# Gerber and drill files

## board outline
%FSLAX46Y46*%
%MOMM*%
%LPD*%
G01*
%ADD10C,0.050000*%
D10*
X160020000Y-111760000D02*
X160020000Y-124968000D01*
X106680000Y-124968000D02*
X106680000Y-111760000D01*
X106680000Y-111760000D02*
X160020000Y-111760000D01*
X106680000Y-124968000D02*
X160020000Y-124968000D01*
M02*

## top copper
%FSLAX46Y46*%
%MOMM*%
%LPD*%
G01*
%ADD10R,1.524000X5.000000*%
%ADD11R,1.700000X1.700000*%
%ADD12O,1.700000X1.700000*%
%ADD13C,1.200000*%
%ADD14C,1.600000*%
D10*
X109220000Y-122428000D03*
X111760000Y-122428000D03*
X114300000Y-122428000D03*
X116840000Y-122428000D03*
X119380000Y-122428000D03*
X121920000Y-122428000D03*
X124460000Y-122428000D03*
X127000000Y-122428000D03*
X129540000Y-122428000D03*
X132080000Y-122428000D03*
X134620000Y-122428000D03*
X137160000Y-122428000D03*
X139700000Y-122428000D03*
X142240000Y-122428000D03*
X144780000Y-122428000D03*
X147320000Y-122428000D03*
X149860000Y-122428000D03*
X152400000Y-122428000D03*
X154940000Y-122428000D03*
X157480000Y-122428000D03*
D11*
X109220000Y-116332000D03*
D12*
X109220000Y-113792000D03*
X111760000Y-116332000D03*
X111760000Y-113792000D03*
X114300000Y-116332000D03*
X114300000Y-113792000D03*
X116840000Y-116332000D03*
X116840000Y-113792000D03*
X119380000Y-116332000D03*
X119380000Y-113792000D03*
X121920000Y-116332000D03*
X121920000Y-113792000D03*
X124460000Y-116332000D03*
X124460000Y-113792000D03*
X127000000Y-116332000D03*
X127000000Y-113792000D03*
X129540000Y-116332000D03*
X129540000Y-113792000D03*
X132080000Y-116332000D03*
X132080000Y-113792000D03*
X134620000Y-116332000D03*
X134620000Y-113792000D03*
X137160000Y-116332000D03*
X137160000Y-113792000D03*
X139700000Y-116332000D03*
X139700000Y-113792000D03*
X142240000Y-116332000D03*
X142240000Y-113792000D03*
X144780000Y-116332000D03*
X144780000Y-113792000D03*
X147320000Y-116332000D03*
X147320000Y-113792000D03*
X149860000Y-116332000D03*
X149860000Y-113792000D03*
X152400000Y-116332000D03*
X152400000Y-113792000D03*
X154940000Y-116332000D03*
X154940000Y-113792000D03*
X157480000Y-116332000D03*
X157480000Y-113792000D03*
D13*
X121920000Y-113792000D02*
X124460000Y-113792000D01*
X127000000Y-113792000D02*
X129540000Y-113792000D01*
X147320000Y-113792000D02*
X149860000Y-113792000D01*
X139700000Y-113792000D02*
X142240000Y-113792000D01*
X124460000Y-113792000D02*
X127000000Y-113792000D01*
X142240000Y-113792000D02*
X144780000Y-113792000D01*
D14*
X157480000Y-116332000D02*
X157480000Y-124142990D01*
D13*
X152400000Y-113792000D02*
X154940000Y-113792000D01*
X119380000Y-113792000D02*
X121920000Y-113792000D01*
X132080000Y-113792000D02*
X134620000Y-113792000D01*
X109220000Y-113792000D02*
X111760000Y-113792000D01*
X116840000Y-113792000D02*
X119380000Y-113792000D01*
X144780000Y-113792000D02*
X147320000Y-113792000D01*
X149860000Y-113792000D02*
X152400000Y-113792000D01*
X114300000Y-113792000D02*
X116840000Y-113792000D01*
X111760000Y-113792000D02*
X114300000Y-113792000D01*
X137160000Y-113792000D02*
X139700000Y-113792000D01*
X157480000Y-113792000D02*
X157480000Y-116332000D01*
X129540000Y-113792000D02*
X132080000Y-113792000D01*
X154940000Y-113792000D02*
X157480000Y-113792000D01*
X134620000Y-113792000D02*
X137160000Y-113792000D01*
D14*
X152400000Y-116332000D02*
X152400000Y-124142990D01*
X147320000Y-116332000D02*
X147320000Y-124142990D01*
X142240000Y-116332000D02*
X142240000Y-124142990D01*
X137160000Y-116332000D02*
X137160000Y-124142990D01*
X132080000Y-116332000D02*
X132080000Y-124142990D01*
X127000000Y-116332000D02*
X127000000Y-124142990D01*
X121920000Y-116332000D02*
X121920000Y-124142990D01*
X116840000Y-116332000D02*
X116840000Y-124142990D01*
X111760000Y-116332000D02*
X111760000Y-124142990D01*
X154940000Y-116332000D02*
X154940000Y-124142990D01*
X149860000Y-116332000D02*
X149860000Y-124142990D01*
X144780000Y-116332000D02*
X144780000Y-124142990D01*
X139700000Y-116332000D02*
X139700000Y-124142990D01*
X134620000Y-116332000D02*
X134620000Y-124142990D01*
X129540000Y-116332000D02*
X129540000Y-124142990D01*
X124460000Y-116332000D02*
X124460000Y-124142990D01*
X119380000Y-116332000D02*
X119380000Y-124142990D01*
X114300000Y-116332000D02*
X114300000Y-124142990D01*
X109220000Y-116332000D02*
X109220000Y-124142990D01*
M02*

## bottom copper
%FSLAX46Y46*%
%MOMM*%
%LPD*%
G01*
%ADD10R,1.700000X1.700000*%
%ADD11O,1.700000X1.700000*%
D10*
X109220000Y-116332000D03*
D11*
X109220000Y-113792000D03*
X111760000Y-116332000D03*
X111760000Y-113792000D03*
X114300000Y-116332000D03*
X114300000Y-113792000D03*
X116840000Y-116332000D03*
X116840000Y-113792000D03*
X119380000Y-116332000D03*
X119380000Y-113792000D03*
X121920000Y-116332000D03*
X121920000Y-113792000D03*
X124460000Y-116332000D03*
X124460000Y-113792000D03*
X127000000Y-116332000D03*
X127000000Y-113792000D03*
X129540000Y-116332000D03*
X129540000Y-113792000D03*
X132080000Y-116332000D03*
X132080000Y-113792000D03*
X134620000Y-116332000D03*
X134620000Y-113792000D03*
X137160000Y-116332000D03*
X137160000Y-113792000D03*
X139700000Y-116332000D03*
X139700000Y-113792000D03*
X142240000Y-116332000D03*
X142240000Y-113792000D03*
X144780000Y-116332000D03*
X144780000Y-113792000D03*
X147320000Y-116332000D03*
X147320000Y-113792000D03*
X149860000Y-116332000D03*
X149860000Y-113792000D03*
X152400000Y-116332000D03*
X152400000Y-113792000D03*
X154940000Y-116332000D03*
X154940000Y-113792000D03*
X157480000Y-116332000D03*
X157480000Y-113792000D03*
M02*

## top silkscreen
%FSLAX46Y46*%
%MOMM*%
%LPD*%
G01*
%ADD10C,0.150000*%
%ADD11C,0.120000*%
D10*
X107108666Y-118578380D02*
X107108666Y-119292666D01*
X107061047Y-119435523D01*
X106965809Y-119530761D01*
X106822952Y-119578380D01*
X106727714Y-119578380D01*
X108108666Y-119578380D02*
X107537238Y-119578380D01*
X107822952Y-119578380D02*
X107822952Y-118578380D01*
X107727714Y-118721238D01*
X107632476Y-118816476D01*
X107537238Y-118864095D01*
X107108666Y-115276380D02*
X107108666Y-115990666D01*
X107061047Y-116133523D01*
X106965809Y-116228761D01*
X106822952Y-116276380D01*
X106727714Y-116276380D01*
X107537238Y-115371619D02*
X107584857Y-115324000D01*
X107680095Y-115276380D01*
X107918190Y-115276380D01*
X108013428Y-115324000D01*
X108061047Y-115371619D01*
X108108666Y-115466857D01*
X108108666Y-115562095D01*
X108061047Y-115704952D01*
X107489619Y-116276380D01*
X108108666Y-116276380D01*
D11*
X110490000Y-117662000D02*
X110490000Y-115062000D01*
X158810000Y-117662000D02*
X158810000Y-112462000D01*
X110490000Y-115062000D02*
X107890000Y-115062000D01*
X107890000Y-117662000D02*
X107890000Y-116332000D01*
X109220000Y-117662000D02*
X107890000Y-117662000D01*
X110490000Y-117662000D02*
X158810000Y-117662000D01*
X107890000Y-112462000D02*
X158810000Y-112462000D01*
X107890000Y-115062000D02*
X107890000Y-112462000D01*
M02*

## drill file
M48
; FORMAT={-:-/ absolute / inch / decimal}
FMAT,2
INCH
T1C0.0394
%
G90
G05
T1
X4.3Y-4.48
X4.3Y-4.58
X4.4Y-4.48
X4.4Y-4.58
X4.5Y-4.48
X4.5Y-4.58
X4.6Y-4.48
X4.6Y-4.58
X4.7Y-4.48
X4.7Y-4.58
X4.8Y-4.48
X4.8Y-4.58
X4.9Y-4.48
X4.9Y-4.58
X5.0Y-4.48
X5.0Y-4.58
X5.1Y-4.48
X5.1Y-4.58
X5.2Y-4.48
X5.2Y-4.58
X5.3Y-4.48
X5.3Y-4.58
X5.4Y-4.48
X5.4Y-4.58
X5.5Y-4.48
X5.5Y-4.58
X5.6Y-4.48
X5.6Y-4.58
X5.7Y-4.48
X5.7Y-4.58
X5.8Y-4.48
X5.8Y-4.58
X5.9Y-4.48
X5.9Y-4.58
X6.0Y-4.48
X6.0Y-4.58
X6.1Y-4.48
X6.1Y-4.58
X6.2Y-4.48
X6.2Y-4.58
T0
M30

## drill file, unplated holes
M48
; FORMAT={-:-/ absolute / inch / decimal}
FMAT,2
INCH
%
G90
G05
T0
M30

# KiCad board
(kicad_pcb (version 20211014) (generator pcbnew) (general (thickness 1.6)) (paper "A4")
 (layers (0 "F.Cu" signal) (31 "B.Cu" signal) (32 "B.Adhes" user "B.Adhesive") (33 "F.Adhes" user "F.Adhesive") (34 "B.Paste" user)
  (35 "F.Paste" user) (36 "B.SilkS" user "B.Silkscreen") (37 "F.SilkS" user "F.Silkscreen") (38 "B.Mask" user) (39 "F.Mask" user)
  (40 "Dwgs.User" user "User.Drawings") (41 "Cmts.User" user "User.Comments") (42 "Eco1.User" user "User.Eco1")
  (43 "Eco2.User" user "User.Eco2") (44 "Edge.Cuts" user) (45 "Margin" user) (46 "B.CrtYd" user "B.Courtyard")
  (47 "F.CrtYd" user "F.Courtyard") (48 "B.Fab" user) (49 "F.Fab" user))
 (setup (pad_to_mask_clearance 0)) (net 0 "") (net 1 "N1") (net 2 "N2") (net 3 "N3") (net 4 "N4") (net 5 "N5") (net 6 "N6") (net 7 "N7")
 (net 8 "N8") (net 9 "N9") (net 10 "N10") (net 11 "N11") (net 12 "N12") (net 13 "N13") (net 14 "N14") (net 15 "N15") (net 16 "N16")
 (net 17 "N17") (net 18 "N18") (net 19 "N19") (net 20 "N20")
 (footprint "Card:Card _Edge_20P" (layer "F.Cu") (at 116.84 124.968)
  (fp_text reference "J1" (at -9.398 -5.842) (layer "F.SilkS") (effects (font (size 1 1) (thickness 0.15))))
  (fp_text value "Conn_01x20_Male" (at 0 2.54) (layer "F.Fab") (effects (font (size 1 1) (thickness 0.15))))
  (pad "1" smd rect locked (at -7.62 -2.54) (size 1.524 5) (layers "F.Cu" "F.Paste" "F.Mask") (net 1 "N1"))
  (pad "2" smd rect locked (at -5.08 -2.54) (size 1.524 5) (layers "F.Cu" "F.Paste" "F.Mask") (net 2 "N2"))
  (pad "3" smd rect locked (at -2.54 -2.54) (size 1.524 5) (layers "F.Cu" "F.Paste" "F.Mask") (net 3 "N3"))
  (pad "4" smd rect locked (at 0 -2.54) (size 1.524 5) (layers "F.Cu" "F.Paste" "F.Mask") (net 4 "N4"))
  (pad "5" smd rect locked (at 2.54 -2.54) (size 1.524 5) (layers "F.Cu" "F.Paste" "F.Mask") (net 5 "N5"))
  (pad "6" smd rect locked (at 5.08 -2.54) (size 1.524 5) (layers "F.Cu" "F.Paste" "F.Mask") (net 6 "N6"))
  (pad "7" smd rect locked (at 7.62 -2.54) (size 1.524 5) (layers "F.Cu" "F.Paste" "F.Mask") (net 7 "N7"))
  (pad "8" smd rect locked (at 10.16 -2.54) (size 1.524 5) (layers "F.Cu" "F.Paste" "F.Mask") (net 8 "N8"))
  (pad "9" smd rect locked (at 12.7 -2.54) (size 1.524 5) (layers "F.Cu" "F.Paste" "F.Mask") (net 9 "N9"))
  (pad "10" smd rect locked (at 15.24 -2.54) (size 1.524 5) (layers "F.Cu" "F.Paste" "F.Mask") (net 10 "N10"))
  (pad "11" smd rect locked (at 17.78 -2.54) (size 1.524 5) (layers "F.Cu" "F.Paste" "F.Mask") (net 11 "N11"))
  (pad "12" smd rect locked (at 20.32 -2.54) (size 1.524 5) (layers "F.Cu" "F.Paste" "F.Mask") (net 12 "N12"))
  (pad "13" smd rect locked (at 22.86 -2.54) (size 1.524 5) (layers "F.Cu" "F.Paste" "F.Mask") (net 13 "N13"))
  (pad "14" smd rect locked (at 25.4 -2.54) (size 1.524 5) (layers "F.Cu" "F.Paste" "F.Mask") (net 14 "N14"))
  (pad "15" smd rect locked (at 27.94 -2.54) (size 1.524 5) (layers "F.Cu" "F.Paste" "F.Mask") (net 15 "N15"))
  (pad "16" smd rect locked (at 30.48 -2.54) (size 1.524 5) (layers "F.Cu" "F.Paste" "F.Mask") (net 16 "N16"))
  (pad "17" smd rect locked (at 33.02 -2.54) (size 1.524 5) (layers "F.Cu" "F.Paste" "F.Mask") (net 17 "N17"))
  (pad "18" smd rect locked (at 35.56 -2.54) (size 1.524 5) (layers "F.Cu" "F.Paste" "F.Mask") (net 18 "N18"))
  (pad "19" smd rect locked (at 38.1 -2.54) (size 1.524 5) (layers "F.Cu" "F.Paste" "F.Mask") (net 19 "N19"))
  (pad "20" smd rect locked (at 40.64 -2.54) (size 1.524 5) (layers "F.Cu" "F.Paste" "F.Mask") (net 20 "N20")))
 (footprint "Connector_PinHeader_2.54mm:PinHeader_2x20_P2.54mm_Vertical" (layer "F.Cu") (at 109.22 116.332 90)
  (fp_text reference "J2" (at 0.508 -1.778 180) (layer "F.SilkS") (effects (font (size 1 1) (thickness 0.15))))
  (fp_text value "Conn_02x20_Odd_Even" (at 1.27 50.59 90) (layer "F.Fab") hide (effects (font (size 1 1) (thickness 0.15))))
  (fp_line (start -1.33 1.27) (end 1.27 1.27) (layer "F.SilkS") (width 0.12))
  (fp_line (start -1.33 49.59) (end 3.87 49.59) (layer "F.SilkS") (width 0.12))
  (fp_line (start 1.27 1.27) (end 1.27 -1.33) (layer "F.SilkS") (width 0.12))
  (fp_line (start -1.33 -1.33) (end 0 -1.33) (layer "F.SilkS") (width 0.12))
  (fp_line (start -1.33 0) (end -1.33 -1.33) (layer "F.SilkS") (width 0.12))
  (fp_line (start -1.33 1.27) (end -1.33 49.59) (layer "F.SilkS") (width 0.12))
  (fp_line (start 3.87 -1.33) (end 3.87 49.59) (layer "F.SilkS") (width 0.12))
  (fp_line (start 1.27 -1.33) (end 3.87 -1.33) (layer "F.SilkS") (width 0.12))
  (pad "1" thru_hole rect locked (at 0 0 90) (size 1.7 1.7) (drill 1) (layers *.Cu *.Mask) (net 1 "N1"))
  (pad "2" thru_hole oval locked (at 2.54 0 90) (size 1.7 1.7) (drill 1) (layers *.Cu *.Mask) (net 20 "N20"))
  (pad "3" thru_hole oval locked (at 0 2.54 90) (size 1.7 1.7) (drill 1) (layers *.Cu *.Mask) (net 2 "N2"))
  (pad "4" thru_hole oval locked (at 2.54 2.54 90) (size 1.7 1.7) (drill 1) (layers *.Cu *.Mask) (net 20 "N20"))
  (pad "5" thru_hole oval locked (at 0 5.08 90) (size 1.7 1.7) (drill 1) (layers *.Cu *.Mask) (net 3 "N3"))
  (pad "6" thru_hole oval locked (at 2.54 5.08 90) (size 1.7 1.7) (drill 1) (layers *.Cu *.Mask) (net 20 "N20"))
  (pad "7" thru_hole oval locked (at 0 7.62 90) (size 1.7 1.7) (drill 1) (layers *.Cu *.Mask) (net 4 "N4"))
  (pad "8" thru_hole oval locked (at 2.54 7.62 90) (size 1.7 1.7) (drill 1) (layers *.Cu *.Mask) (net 20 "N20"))
  (pad "9" thru_hole oval locked (at 0 10.16 90) (size 1.7 1.7) (drill 1) (layers *.Cu *.Mask) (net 5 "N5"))
  (pad "10" thru_hole oval locked (at 2.54 10.16 90) (size 1.7 1.7) (drill 1) (layers *.Cu *.Mask) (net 20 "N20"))
  (pad "11" thru_hole oval locked (at 0 12.7 90) (size 1.7 1.7) (drill 1) (layers *.Cu *.Mask) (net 6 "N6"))
  (pad "12" thru_hole oval locked (at 2.54 12.7 90) (size 1.7 1.7) (drill 1) (layers *.Cu *.Mask) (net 20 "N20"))
  (pad "13" thru_hole oval locked (at 0 15.24 90) (size 1.7 1.7) (drill 1) (layers *.Cu *.Mask) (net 7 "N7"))
  (pad "14" thru_hole oval locked (at 2.54 15.24 90) (size 1.7 1.7) (drill 1) (layers *.Cu *.Mask) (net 20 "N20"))
  (pad "15" thru_hole oval locked (at 0 17.78 90) (size 1.7 1.7) (drill 1) (layers *.Cu *.Mask) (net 8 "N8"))
  (pad "16" thru_hole oval locked (at 2.54 17.78 90) (size 1.7 1.7) (drill 1) (layers *.Cu *.Mask) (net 20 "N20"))
  (pad "17" thru_hole oval locked (at 0 20.32 90) (size 1.7 1.7) (drill 1) (layers *.Cu *.Mask) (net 9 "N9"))
  (pad "18" thru_hole oval locked (at 2.54 20.32 90) (size 1.7 1.7) (drill 1) (layers *.Cu *.Mask) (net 20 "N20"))
  (pad "19" thru_hole oval locked (at 0 22.86 90) (size 1.7 1.7) (drill 1) (layers *.Cu *.Mask) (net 10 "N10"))
  (pad "20" thru_hole oval locked (at 2.54 22.86 90) (size 1.7 1.7) (drill 1) (layers *.Cu *.Mask) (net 20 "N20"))
  (pad "21" thru_hole oval locked (at 0 25.4 90) (size 1.7 1.7) (drill 1) (layers *.Cu *.Mask) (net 11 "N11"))
  (pad "22" thru_hole oval locked (at 2.54 25.4 90) (size 1.7 1.7) (drill 1) (layers *.Cu *.Mask) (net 20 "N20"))
  (pad "23" thru_hole oval locked (at 0 27.94 90) (size 1.7 1.7) (drill 1) (layers *.Cu *.Mask) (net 12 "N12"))
  (pad "24" thru_hole oval locked (at 2.54 27.94 90) (size 1.7 1.7) (drill 1) (layers *.Cu *.Mask) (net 20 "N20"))
  (pad "25" thru_hole oval locked (at 0 30.48 90) (size 1.7 1.7) (drill 1) (layers *.Cu *.Mask) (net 13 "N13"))
  (pad "26" thru_hole oval locked (at 2.54 30.48 90) (size 1.7 1.7) (drill 1) (layers *.Cu *.Mask) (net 20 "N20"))
  (pad "27" thru_hole oval locked (at 0 33.02 90) (size 1.7 1.7) (drill 1) (layers *.Cu *.Mask) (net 14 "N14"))
  (pad "28" thru_hole oval locked (at 2.54 33.02 90) (size 1.7 1.7) (drill 1) (layers *.Cu *.Mask) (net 20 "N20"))
  (pad "29" thru_hole oval locked (at 0 35.56 90) (size 1.7 1.7) (drill 1) (layers *.Cu *.Mask) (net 15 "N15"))
  (pad "30" thru_hole oval locked (at 2.54 35.56 90) (size 1.7 1.7) (drill 1) (layers *.Cu *.Mask) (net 20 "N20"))
  (pad "31" thru_hole oval locked (at 0 38.1 90) (size 1.7 1.7) (drill 1) (layers *.Cu *.Mask) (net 16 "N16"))
  (pad "32" thru_hole oval locked (at 2.54 38.1 90) (size 1.7 1.7) (drill 1) (layers *.Cu *.Mask) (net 20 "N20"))
  (pad "33" thru_hole oval locked (at 0 40.64 90) (size 1.7 1.7) (drill 1) (layers *.Cu *.Mask) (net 17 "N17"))
  (pad "34" thru_hole oval locked (at 2.54 40.64 90) (size 1.7 1.7) (drill 1) (layers *.Cu *.Mask) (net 20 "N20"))
  (pad "35" thru_hole oval locked (at 0 43.18 90) (size 1.7 1.7) (drill 1) (layers *.Cu *.Mask) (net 18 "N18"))
  (pad "36" thru_hole oval locked (at 2.54 43.18 90) (size 1.7 1.7) (drill 1) (layers *.Cu *.Mask) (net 20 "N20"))
  (pad "37" thru_hole oval locked (at 0 45.72 90) (size 1.7 1.7) (drill 1) (layers *.Cu *.Mask) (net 19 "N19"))
  (pad "38" thru_hole oval locked (at 2.54 45.72 90) (size 1.7 1.7) (drill 1) (layers *.Cu *.Mask) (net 20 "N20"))
  (pad "39" thru_hole oval locked (at 0 48.26 90) (size 1.7 1.7) (drill 1) (layers *.Cu *.Mask) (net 20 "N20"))
  (pad "40" thru_hole oval locked (at 2.54 48.26 90) (size 1.7 1.7) (drill 1) (layers *.Cu *.Mask) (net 20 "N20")))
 (gr_line (start 160.02 111.76) (end 160.02 124.968) (layer "Edge.Cuts") (width 0.05))
 (gr_line (start 106.68 124.968) (end 106.68 111.76) (layer "Edge.Cuts") (width 0.05))
 (gr_line (start 106.68 111.76) (end 160.02 111.76) (layer "Edge.Cuts") (width 0.05))
 (gr_line (start 106.68 124.968) (end 160.02 124.968) (layer "Edge.Cuts") (width 0.05))
 (segment (start 121.92 113.792) (end 124.46 113.792) (width 1.2) (layer "F.Cu") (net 20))
 (segment (start 127 113.792) (end 129.54 113.792) (width 1.2) (layer "F.Cu") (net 20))
 (segment (start 147.32 113.792) (end 149.86 113.792) (width 1.2) (layer "F.Cu") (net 20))
 (segment (start 139.7 113.792) (end 142.24 113.792) (width 1.2) (layer "F.Cu") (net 20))
 (segment (start 124.46 113.792) (end 127 113.792) (width 1.2) (layer "F.Cu") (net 20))
 (segment (start 142.24 113.792) (end 144.78 113.792) (width 1.2) (layer "F.Cu") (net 20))
 (segment (start 157.48 116.332) (end 157.48 124.14299) (width 1.6) (layer "F.Cu") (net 20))
 (segment (start 152.4 113.792) (end 154.94 113.792) (width 1.2) (layer "F.Cu") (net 20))
 (segment (start 119.38 113.792) (end 121.92 113.792) (width 1.2) (layer "F.Cu") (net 20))
 (segment (start 132.08 113.792) (end 134.62 113.792) (width 1.2) (layer "F.Cu") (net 20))
 (segment (start 109.22 113.792) (end 111.76 113.792) (width 1.2) (layer "F.Cu") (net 20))
 (segment (start 116.84 113.792) (end 119.38 113.792) (width 1.2) (layer "F.Cu") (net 20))
 (segment (start 144.78 113.792) (end 147.32 113.792) (width 1.2) (layer "F.Cu") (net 20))
 (segment (start 149.86 113.792) (end 152.4 113.792) (width 1.2) (layer "F.Cu") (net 20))
 (segment (start 114.3 113.792) (end 116.84 113.792) (width 1.2) (layer "F.Cu") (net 20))
 (segment (start 111.76 113.792) (end 114.3 113.792) (width 1.2) (layer "F.Cu") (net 20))
 (segment (start 137.16 113.792) (end 139.7 113.792) (width 1.2) (layer "F.Cu") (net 20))
 (segment (start 157.48 113.792) (end 157.48 116.332) (width 1.2) (layer "F.Cu") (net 20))
 (segment (start 129.54 113.792) (end 132.08 113.792) (width 1.2) (layer "F.Cu") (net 20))
 (segment (start 154.94 113.792) (end 157.48 113.792) (width 1.2) (layer "F.Cu") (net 20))
 (segment (start 134.62 113.792) (end 137.16 113.792) (width 1.2) (layer "F.Cu") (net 20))
 (segment (start 152.4 116.332) (end 152.4 124.14299) (width 1.6) (layer "F.Cu") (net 18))
 (segment (start 147.32 116.332) (end 147.32 124.14299) (width 1.6) (layer "F.Cu") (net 16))
 (segment (start 142.24 116.332) (end 142.24 124.14299) (width 1.6) (layer "F.Cu") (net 14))
 (segment (start 137.16 116.332) (end 137.16 124.14299) (width 1.6) (layer "F.Cu") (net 12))
 (segment (start 132.08 116.332) (end 132.08 124.14299) (width 1.6) (layer "F.Cu") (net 10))
 (segment (start 127 116.332) (end 127 124.14299) (width 1.6) (layer "F.Cu") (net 8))
 (segment (start 121.92 116.332) (end 121.92 124.14299) (width 1.6) (layer "F.Cu") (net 6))
 (segment (start 116.84 116.332) (end 116.84 124.14299) (width 1.6) (layer "F.Cu") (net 4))
 (segment (start 111.76 116.332) (end 111.76 124.14299) (width 1.6) (layer "F.Cu") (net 2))
 (segment (start 154.94 116.332) (end 154.94 124.14299) (width 1.6) (layer "F.Cu") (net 19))
 (segment (start 149.86 116.332) (end 149.86 124.14299) (width 1.6) (layer "F.Cu") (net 17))
 (segment (start 144.78 116.332) (end 144.78 124.14299) (width 1.6) (layer "F.Cu") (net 15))
 (segment (start 139.7 116.332) (end 139.7 124.14299) (width 1.6) (layer "F.Cu") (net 13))
 (segment (start 134.62 116.332) (end 134.62 124.14299) (width 1.6) (layer "F.Cu") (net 11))
 (segment (start 129.54 116.332) (end 129.54 124.14299) (width 1.6) (layer "F.Cu") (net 9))
 (segment (start 124.46 116.332) (end 124.46 124.14299) (width 1.6) (layer "F.Cu") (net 7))
 (segment (start 119.38 116.332) (end 119.38 124.14299) (width 1.6) (layer "F.Cu") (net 5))
 (segment (start 114.3 116.332) (end 114.3 124.14299) (width 1.6) (layer "F.Cu") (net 3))
 (segment (start 109.22 116.332) (end 109.22 124.14299) (width 1.6) (layer "F.Cu") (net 1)))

